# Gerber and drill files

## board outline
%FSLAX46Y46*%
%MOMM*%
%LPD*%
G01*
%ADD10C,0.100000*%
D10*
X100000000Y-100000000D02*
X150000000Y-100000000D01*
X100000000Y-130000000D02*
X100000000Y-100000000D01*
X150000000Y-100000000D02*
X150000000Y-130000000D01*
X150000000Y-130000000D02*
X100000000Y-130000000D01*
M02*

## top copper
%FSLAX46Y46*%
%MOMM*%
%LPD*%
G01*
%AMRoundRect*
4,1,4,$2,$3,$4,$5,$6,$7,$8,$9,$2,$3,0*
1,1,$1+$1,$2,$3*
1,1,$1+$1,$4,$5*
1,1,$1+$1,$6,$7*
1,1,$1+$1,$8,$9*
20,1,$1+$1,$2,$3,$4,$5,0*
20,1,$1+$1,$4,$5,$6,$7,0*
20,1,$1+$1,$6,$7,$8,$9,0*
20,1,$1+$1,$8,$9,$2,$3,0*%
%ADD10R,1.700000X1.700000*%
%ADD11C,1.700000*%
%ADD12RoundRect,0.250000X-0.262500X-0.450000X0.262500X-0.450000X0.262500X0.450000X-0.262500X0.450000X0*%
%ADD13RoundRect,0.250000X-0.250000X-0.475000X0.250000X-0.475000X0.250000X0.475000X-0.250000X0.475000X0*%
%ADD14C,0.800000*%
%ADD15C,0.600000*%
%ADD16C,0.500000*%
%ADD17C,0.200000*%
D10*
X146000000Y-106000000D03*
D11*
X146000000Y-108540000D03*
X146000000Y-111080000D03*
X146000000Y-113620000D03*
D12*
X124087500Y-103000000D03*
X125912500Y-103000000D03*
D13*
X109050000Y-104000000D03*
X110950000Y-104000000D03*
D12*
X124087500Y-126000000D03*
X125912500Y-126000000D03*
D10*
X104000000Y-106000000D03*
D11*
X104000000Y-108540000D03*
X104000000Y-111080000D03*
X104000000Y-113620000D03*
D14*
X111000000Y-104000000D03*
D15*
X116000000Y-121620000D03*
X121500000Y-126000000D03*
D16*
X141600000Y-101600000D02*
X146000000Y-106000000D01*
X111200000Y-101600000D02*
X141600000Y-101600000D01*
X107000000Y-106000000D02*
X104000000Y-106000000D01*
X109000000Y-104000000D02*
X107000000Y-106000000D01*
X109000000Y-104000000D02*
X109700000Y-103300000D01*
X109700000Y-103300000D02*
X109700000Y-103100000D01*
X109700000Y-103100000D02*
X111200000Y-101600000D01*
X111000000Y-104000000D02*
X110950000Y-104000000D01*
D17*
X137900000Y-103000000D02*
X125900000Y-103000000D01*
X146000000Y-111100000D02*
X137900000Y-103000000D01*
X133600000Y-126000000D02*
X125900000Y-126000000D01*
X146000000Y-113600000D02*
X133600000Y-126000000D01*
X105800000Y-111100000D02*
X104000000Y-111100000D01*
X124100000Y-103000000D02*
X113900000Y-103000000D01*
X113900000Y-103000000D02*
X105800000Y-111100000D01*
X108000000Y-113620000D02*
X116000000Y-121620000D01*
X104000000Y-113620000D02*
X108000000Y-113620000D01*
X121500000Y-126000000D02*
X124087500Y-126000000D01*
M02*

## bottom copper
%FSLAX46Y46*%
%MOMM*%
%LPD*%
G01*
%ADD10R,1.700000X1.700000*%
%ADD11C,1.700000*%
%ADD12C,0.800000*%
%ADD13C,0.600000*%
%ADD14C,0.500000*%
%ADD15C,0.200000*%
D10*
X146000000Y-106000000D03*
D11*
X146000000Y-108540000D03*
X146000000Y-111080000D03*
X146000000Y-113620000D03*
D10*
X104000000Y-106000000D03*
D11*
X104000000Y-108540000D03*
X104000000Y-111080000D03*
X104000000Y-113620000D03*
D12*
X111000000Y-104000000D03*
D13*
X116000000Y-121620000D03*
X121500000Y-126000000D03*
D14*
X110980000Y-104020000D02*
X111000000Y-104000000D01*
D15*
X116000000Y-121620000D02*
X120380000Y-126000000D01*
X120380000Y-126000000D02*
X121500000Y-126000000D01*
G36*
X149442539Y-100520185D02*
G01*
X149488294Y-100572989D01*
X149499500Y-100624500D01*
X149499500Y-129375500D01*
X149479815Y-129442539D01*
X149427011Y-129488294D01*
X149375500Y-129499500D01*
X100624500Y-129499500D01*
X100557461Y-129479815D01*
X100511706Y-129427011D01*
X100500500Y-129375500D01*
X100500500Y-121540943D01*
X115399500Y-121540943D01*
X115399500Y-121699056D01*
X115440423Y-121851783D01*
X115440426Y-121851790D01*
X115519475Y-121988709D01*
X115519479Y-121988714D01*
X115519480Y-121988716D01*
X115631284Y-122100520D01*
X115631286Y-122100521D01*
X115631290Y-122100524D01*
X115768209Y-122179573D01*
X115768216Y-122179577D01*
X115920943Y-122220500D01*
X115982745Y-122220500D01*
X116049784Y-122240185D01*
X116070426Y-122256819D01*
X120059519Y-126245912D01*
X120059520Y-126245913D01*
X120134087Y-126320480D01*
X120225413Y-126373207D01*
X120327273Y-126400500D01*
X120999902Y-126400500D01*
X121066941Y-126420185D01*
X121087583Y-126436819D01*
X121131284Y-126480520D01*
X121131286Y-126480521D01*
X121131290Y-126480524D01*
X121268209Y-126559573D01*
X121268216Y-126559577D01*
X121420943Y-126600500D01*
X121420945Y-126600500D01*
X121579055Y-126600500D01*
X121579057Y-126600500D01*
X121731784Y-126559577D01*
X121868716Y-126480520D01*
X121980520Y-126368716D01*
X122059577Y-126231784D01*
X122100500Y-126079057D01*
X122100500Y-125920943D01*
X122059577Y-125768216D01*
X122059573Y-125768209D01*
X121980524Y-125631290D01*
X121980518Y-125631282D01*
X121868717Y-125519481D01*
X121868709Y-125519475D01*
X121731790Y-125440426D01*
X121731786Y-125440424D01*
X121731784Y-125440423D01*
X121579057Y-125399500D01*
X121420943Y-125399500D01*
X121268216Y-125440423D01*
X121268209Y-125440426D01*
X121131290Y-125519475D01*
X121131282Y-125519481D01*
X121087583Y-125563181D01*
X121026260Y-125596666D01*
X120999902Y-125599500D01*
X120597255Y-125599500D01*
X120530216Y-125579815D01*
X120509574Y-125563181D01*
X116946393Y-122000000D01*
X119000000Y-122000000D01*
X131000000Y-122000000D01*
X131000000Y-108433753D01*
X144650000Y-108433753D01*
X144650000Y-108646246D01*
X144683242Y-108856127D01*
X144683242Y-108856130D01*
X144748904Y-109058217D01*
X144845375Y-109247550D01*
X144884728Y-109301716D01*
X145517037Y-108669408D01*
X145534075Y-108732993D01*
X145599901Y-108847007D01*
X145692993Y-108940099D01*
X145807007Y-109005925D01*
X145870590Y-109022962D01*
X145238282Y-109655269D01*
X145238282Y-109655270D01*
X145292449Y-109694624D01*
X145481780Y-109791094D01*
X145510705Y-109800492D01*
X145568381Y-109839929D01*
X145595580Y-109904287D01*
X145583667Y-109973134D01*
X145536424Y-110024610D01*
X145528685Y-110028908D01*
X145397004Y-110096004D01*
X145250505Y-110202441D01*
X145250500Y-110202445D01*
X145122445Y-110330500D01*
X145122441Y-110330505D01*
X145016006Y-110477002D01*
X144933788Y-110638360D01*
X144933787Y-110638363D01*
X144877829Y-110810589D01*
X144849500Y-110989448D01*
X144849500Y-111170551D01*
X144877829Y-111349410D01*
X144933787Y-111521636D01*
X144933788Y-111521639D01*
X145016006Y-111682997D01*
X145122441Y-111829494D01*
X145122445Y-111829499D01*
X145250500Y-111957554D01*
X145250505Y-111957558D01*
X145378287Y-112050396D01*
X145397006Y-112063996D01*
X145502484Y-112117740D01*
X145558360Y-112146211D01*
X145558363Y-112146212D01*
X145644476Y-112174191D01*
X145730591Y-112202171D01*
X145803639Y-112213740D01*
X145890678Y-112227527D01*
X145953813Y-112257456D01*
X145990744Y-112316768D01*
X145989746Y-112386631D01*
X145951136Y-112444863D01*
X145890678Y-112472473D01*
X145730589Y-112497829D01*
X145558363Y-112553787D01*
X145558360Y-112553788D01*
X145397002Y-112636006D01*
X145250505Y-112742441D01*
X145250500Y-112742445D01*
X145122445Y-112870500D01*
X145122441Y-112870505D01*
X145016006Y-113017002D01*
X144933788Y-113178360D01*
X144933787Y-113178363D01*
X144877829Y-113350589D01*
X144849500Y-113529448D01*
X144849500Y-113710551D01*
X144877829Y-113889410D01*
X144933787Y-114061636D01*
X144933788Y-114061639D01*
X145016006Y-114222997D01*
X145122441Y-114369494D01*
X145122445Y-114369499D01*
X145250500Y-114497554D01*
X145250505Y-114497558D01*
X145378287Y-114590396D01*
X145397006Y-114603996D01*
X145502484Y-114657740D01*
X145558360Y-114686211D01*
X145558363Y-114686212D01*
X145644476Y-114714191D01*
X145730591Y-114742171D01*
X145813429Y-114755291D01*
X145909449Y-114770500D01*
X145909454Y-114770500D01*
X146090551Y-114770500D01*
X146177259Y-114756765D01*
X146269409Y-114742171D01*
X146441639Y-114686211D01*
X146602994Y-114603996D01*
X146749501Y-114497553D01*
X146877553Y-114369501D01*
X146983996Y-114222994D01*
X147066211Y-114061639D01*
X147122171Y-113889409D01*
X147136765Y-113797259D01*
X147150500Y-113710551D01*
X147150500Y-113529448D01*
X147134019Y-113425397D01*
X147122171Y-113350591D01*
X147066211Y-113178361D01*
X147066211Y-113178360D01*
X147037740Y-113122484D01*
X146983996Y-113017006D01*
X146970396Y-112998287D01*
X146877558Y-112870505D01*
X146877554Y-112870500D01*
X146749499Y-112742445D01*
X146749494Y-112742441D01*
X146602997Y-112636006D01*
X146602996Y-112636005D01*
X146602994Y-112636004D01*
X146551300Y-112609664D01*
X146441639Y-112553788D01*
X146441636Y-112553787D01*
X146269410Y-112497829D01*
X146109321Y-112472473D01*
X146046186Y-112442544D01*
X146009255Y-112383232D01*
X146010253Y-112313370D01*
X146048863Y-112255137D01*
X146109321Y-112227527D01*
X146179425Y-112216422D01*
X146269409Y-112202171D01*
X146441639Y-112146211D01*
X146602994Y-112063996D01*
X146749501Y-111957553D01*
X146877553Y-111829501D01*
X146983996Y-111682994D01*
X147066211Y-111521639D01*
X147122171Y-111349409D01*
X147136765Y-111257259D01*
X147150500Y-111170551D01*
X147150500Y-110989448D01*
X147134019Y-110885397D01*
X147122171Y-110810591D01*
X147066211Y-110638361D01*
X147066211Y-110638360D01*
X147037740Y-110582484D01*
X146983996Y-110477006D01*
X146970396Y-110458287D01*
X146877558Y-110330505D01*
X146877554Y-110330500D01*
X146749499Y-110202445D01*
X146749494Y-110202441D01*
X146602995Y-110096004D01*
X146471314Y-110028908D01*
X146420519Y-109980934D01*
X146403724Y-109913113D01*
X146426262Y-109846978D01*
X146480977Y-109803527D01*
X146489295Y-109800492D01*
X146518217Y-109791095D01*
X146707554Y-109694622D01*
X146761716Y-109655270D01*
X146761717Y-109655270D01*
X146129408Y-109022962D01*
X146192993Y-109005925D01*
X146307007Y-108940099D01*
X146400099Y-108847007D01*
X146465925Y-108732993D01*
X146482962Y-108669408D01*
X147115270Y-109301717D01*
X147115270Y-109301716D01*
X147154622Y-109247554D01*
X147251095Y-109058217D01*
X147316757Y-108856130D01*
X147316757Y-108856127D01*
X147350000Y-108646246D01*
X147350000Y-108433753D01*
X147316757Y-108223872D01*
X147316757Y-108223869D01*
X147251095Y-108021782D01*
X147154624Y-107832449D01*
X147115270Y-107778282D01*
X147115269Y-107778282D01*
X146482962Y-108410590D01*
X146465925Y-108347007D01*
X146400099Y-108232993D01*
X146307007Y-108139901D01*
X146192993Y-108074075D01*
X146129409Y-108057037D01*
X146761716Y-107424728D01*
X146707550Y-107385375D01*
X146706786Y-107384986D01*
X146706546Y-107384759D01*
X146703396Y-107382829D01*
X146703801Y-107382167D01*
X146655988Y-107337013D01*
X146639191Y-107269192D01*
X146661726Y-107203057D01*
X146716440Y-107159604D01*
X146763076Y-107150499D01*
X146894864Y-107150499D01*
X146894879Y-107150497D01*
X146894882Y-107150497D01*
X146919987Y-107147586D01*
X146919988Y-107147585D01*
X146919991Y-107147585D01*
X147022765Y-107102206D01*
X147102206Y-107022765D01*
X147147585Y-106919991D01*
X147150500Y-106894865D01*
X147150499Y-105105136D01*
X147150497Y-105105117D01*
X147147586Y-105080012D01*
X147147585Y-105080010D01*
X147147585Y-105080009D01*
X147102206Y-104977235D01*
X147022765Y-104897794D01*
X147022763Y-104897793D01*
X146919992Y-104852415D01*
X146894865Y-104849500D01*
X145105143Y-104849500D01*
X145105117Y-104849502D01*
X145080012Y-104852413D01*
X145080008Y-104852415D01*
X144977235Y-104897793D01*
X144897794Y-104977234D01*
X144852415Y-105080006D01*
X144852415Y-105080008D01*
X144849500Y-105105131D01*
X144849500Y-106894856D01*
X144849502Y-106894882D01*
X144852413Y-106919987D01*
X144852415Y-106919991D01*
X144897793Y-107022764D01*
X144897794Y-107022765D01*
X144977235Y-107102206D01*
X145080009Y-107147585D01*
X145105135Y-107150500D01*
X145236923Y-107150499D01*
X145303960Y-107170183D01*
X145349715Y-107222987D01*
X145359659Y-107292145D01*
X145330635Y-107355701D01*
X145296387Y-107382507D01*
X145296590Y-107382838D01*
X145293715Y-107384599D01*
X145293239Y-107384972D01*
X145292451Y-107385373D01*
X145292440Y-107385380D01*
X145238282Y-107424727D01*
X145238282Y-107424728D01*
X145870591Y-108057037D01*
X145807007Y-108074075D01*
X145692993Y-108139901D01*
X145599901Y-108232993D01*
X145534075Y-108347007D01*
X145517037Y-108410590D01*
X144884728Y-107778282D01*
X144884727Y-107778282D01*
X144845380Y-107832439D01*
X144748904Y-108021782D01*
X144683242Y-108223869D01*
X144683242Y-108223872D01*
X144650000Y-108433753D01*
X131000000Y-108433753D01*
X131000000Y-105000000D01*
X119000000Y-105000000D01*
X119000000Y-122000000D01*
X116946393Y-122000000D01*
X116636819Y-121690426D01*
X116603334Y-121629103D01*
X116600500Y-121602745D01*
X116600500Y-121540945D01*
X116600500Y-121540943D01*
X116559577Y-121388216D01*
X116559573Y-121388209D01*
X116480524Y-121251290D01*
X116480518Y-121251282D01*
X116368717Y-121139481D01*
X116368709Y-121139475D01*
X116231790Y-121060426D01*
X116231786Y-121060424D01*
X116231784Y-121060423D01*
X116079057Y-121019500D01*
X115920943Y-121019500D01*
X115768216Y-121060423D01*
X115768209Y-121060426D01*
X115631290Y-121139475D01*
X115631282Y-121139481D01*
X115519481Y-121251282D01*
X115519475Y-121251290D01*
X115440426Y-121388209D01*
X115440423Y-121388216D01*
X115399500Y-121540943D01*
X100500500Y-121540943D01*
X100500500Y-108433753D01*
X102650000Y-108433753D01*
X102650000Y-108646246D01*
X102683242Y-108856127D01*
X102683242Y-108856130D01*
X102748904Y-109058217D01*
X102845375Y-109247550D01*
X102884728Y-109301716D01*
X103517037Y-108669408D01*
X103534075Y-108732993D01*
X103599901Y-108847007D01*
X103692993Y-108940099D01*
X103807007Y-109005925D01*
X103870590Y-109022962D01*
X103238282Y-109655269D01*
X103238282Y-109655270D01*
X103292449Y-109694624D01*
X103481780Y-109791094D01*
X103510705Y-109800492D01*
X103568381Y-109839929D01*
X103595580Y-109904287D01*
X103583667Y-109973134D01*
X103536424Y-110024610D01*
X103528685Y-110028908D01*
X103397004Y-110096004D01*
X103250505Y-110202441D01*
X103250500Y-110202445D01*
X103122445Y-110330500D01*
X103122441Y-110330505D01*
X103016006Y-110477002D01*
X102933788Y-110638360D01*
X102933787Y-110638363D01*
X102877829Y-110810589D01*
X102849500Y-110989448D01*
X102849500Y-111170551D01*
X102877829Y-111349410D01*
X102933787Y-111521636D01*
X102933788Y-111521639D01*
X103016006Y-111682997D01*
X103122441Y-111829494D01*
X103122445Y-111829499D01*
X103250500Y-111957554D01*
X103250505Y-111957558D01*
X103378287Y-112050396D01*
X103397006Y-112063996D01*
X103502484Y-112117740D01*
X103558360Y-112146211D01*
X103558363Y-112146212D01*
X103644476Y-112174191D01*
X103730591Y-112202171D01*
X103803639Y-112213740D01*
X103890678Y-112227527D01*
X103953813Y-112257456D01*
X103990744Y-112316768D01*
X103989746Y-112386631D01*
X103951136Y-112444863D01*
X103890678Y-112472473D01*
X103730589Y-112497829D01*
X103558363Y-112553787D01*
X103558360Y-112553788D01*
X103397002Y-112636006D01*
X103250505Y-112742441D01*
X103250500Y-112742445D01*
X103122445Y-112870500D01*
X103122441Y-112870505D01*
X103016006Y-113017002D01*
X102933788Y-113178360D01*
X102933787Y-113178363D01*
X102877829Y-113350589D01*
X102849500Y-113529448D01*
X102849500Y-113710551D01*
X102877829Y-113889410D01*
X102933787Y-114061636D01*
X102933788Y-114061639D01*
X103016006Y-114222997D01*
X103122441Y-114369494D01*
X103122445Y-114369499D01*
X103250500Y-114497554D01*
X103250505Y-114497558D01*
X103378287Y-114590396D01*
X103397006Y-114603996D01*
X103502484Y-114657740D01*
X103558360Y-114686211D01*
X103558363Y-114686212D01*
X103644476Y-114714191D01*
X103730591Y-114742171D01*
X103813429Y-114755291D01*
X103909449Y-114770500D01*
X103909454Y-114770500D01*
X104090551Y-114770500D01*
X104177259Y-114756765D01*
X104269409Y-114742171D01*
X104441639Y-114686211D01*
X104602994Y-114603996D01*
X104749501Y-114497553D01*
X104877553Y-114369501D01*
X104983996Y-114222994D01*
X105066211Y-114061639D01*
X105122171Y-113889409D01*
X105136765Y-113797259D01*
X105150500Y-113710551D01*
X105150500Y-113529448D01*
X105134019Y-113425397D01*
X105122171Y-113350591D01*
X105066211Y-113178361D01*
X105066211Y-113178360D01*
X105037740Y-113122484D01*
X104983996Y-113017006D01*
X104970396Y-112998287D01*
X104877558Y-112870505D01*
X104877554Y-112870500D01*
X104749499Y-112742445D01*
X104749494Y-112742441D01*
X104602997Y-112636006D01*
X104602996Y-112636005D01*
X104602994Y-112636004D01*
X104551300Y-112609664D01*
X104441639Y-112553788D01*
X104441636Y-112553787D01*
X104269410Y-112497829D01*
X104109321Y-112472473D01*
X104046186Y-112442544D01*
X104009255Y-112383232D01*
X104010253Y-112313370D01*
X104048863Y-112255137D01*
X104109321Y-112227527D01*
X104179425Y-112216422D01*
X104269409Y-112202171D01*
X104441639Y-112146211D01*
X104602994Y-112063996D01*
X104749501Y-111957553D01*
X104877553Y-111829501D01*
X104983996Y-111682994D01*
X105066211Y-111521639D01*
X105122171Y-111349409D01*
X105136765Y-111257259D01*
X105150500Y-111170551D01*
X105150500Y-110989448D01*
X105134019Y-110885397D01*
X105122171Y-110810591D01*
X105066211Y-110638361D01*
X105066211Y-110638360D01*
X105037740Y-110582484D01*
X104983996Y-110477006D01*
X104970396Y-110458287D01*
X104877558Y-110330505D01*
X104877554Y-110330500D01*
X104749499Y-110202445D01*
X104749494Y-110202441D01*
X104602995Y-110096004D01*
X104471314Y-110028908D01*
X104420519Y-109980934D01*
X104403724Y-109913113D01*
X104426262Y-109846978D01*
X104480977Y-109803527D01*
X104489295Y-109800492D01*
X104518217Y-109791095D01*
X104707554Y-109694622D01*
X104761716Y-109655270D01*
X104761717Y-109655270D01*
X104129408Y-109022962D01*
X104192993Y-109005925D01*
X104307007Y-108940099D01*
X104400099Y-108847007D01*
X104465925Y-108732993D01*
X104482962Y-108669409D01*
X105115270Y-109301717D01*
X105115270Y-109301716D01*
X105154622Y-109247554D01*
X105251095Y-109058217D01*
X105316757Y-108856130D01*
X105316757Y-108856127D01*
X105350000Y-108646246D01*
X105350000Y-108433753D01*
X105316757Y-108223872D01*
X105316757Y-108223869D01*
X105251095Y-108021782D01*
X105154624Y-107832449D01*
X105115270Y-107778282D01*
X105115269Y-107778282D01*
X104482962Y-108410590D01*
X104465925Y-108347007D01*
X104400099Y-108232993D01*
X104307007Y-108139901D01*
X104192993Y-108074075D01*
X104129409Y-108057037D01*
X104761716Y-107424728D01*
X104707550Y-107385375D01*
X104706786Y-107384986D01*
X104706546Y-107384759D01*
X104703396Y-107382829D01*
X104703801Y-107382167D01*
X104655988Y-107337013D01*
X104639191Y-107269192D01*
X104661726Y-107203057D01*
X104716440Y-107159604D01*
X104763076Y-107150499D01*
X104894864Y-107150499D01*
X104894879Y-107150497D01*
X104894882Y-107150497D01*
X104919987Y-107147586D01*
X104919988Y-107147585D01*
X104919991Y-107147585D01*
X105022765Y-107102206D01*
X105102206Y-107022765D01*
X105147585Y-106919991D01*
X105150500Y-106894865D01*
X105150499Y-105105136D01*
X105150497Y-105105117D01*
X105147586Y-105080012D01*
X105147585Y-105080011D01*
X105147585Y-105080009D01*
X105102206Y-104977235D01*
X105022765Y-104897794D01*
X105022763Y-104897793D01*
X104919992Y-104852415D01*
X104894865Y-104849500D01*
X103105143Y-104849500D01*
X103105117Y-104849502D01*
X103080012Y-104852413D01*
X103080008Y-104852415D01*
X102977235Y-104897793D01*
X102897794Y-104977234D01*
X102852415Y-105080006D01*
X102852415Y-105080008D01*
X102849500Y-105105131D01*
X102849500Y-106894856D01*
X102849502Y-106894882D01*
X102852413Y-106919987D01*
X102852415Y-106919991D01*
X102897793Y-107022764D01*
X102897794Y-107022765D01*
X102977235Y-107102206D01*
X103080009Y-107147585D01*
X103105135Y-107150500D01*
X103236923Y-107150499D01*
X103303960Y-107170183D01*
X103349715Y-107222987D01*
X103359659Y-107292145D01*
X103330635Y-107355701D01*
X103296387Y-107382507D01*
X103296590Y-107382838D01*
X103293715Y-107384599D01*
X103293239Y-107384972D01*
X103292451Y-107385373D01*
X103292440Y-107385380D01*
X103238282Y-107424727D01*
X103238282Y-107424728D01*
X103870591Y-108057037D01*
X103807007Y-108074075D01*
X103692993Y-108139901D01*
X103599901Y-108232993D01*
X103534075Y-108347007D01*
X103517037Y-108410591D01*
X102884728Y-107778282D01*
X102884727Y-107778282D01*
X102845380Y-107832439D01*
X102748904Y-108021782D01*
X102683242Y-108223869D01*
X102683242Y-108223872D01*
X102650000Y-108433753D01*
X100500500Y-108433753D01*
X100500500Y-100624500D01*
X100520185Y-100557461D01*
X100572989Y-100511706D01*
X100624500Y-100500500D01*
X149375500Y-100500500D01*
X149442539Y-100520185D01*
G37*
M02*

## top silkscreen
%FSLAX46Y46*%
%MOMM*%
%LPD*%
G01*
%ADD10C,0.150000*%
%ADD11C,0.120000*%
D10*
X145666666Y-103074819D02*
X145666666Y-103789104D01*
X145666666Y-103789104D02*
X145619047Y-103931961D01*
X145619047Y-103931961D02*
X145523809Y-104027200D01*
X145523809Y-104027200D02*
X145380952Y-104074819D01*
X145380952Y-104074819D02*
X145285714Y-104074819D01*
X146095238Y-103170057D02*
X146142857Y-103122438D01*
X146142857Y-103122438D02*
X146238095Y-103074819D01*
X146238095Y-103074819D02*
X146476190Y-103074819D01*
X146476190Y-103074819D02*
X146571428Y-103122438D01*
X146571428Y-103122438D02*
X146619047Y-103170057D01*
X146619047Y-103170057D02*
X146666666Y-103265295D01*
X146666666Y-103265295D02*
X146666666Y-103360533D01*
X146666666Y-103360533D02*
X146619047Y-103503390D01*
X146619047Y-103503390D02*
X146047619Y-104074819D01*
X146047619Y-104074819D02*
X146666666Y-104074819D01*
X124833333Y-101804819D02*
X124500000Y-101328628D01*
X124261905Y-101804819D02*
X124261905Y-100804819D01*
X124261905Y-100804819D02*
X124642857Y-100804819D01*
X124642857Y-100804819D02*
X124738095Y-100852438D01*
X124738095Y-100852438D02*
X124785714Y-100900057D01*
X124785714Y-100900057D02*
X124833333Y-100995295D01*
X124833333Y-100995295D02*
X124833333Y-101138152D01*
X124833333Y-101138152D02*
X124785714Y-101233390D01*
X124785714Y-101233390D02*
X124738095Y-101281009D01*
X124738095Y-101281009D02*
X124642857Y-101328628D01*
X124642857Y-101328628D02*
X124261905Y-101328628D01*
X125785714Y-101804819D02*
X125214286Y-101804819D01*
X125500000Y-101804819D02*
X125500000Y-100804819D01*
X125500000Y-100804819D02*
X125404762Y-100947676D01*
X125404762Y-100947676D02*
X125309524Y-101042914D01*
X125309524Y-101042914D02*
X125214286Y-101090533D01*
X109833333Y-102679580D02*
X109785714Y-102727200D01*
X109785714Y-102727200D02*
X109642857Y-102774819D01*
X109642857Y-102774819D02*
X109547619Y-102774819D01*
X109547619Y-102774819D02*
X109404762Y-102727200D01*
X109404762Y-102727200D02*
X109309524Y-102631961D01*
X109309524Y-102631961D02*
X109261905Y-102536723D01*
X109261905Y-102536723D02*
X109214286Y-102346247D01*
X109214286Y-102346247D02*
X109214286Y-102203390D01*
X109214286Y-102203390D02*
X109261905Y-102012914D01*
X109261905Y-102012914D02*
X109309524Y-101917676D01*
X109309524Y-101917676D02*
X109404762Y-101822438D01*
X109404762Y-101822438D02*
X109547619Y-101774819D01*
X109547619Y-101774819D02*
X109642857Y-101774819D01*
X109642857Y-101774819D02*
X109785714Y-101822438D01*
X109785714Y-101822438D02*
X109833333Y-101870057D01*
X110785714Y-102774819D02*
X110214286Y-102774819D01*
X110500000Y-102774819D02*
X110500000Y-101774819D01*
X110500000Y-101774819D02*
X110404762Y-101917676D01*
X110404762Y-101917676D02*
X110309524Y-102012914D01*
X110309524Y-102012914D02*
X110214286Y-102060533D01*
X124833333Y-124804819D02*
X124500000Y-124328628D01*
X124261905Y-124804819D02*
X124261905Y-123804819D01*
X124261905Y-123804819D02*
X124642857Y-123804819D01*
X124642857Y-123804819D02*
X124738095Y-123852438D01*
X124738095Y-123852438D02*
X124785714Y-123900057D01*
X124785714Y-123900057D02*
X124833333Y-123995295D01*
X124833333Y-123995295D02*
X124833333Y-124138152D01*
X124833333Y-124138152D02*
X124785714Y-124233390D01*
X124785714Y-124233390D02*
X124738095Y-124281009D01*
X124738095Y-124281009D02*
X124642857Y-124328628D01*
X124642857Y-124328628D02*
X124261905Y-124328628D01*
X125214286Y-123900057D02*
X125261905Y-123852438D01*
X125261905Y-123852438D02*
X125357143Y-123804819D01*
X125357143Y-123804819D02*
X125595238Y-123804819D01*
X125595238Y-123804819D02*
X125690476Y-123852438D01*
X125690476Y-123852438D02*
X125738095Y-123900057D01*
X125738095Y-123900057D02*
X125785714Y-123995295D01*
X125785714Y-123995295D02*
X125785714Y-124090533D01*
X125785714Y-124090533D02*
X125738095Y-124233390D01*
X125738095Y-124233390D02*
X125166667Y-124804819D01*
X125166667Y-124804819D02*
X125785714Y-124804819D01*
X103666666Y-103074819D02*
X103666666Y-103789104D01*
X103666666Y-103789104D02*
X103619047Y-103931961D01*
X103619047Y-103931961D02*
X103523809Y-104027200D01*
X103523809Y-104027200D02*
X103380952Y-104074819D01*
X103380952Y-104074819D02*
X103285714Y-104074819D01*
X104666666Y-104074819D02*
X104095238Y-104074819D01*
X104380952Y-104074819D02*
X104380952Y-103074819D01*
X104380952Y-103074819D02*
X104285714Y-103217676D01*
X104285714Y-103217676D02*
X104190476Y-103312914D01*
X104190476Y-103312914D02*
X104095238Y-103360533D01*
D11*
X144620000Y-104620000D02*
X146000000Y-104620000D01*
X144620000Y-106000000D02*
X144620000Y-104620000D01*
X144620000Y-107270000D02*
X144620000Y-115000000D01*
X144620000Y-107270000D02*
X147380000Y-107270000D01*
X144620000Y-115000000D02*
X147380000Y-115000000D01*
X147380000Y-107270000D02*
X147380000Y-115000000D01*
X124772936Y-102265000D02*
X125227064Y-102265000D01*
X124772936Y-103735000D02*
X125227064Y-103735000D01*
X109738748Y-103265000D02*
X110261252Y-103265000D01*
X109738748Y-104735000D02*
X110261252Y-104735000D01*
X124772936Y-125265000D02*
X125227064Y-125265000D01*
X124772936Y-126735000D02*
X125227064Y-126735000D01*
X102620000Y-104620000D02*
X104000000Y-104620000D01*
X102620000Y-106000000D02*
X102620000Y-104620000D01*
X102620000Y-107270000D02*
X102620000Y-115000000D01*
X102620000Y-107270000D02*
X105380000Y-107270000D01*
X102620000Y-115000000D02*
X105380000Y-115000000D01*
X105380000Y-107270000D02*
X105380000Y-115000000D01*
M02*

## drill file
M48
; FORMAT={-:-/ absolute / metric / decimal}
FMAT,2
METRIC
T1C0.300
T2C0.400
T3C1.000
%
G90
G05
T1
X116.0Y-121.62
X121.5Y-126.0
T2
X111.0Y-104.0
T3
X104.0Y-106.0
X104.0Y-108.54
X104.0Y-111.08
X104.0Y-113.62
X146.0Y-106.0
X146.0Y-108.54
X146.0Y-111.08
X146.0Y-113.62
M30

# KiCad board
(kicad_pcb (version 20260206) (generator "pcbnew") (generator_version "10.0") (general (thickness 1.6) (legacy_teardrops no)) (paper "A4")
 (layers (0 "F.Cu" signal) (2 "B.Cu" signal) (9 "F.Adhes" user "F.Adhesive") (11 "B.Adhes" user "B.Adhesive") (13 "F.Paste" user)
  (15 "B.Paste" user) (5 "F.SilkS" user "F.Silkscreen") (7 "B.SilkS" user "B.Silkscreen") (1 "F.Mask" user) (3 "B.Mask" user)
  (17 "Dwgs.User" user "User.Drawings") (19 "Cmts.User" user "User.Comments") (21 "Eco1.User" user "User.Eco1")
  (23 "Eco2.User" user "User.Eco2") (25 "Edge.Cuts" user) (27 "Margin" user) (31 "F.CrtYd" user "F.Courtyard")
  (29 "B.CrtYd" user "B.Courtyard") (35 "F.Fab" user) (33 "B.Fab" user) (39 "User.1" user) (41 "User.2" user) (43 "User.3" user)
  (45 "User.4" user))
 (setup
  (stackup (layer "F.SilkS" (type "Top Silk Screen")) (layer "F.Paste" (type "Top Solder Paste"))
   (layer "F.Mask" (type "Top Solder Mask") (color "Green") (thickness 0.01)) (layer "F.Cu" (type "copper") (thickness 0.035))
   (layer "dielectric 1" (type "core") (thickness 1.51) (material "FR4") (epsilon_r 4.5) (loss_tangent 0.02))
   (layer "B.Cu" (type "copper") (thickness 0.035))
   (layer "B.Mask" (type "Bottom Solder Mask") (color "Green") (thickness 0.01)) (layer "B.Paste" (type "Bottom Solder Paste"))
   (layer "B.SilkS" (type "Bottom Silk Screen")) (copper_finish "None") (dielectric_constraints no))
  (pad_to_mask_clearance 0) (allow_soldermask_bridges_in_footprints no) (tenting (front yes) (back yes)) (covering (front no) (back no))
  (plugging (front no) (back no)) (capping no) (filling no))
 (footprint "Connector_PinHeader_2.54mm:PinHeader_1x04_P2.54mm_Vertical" (layer "F.Cu") (at 146 106)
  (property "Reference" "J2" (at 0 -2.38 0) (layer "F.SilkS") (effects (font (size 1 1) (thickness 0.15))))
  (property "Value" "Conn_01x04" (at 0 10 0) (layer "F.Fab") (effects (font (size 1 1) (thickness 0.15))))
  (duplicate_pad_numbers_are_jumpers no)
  (fp_line (start -1.38 -1.38) (end 0 -1.38) (stroke (width 0.12) (type solid)) (layer "F.SilkS"))
  (fp_line (start -1.38 0) (end -1.38 -1.38) (stroke (width 0.12) (type solid)) (layer "F.SilkS"))
  (fp_line (start -1.38 1.27) (end -1.38 9) (stroke (width 0.12) (type solid)) (layer "F.SilkS"))
  (fp_line (start -1.38 1.27) (end 1.38 1.27) (stroke (width 0.12) (type solid)) (layer "F.SilkS"))
  (fp_line (start -1.38 9) (end 1.38 9) (stroke (width 0.12) (type solid)) (layer "F.SilkS"))
  (fp_line (start 1.38 1.27) (end 1.38 9) (stroke (width 0.12) (type solid)) (layer "F.SilkS"))
  (pad "1" thru_hole rect (at 0 0) (size 1.7 1.7) (drill 1) (layers "*.Cu" "*.Mask") (remove_unused_layers no) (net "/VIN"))
  (pad "2" thru_hole circle (at 0 2.54) (size 1.7 1.7) (drill 1) (layers "*.Cu" "*.Mask") (remove_unused_layers no) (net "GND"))
  (pad "3" thru_hole circle (at 0 5.08) (size 1.7 1.7) (drill 1) (layers "*.Cu" "*.Mask") (remove_unused_layers no) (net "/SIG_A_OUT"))
  (pad "4" thru_hole circle (at 0 7.62) (size 1.7 1.7) (drill 1) (layers "*.Cu" "*.Mask") (remove_unused_layers no) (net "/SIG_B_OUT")))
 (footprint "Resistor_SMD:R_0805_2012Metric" (layer "F.Cu") (at 125 103)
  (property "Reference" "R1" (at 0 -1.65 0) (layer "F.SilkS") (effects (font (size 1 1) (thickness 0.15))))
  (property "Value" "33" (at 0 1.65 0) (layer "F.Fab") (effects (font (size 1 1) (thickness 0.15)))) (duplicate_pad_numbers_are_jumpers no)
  (fp_line (start -0.227064 -0.735) (end 0.227064 -0.735) (stroke (width 0.12) (type solid)) (layer "F.SilkS"))
  (fp_line (start -0.227064 0.735) (end 0.227064 0.735) (stroke (width 0.12) (type solid)) (layer "F.SilkS"))
  (pad "1" smd roundrect (at -0.9125 0) (size 1.025 1.4) (layers "F.Cu" "F.Mask" "F.Paste") (roundrect_rratio 0.243902) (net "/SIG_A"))
  (pad "2" smd roundrect (at 0.9125 0) (size 1.025 1.4) (layers "F.Cu" "F.Mask" "F.Paste") (roundrect_rratio 0.243902) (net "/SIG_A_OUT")))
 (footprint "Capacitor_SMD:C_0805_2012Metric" (layer "F.Cu") (at 110 104)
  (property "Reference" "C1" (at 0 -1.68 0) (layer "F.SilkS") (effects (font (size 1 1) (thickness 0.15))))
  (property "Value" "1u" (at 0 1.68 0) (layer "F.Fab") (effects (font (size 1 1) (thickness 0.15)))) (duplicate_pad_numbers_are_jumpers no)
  (fp_line (start -0.261252 -0.735) (end 0.261252 -0.735) (stroke (width 0.12) (type solid)) (layer "F.SilkS"))
  (fp_line (start -0.261252 0.735) (end 0.261252 0.735) (stroke (width 0.12) (type solid)) (layer "F.SilkS"))
  (pad "1" smd roundrect (at -0.95 0) (size 1 1.45) (layers "F.Cu" "F.Mask" "F.Paste") (roundrect_rratio 0.25) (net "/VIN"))
  (pad "2" smd roundrect (at 0.95 0) (size 1 1.45) (layers "F.Cu" "F.Mask" "F.Paste") (roundrect_rratio 0.25) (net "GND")))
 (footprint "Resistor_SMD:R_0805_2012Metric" (layer "F.Cu") (at 125 126)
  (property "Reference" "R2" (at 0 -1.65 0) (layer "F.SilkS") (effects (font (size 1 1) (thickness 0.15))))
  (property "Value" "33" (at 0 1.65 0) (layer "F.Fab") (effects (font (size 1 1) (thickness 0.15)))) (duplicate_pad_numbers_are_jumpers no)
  (fp_line (start -0.227064 -0.735) (end 0.227064 -0.735) (stroke (width 0.12) (type solid)) (layer "F.SilkS"))
  (fp_line (start -0.227064 0.735) (end 0.227064 0.735) (stroke (width 0.12) (type solid)) (layer "F.SilkS"))
  (pad "1" smd roundrect (at -0.9125 0) (size 1.025 1.4) (layers "F.Cu" "F.Mask" "F.Paste") (roundrect_rratio 0.243902) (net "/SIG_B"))
  (pad "2" smd roundrect (at 0.9125 0) (size 1.025 1.4) (layers "F.Cu" "F.Mask" "F.Paste") (roundrect_rratio 0.243902) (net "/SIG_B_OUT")))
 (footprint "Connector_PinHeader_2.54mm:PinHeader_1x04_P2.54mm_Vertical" (layer "F.Cu") (at 104 106)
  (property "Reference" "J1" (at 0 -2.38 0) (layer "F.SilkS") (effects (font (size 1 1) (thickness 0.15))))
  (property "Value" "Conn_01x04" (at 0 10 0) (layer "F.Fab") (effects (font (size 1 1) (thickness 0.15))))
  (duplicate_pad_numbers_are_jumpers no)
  (fp_line (start -1.38 -1.38) (end 0 -1.38) (stroke (width 0.12) (type solid)) (layer "F.SilkS"))
  (fp_line (start -1.38 0) (end -1.38 -1.38) (stroke (width 0.12) (type solid)) (layer "F.SilkS"))
  (fp_line (start -1.38 1.27) (end -1.38 9) (stroke (width 0.12) (type solid)) (layer "F.SilkS"))
  (fp_line (start -1.38 1.27) (end 1.38 1.27) (stroke (width 0.12) (type solid)) (layer "F.SilkS"))
  (fp_line (start -1.38 9) (end 1.38 9) (stroke (width 0.12) (type solid)) (layer "F.SilkS"))
  (fp_line (start 1.38 1.27) (end 1.38 9) (stroke (width 0.12) (type solid)) (layer "F.SilkS"))
  (pad "1" thru_hole rect (at 0 0) (size 1.7 1.7) (drill 1) (layers "*.Cu" "*.Mask") (remove_unused_layers no) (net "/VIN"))
  (pad "2" thru_hole circle (at 0 2.54) (size 1.7 1.7) (drill 1) (layers "*.Cu" "*.Mask") (remove_unused_layers no) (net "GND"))
  (pad "3" thru_hole circle (at 0 5.08) (size 1.7 1.7) (drill 1) (layers "*.Cu" "*.Mask") (remove_unused_layers no) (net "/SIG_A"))
  (pad "4" thru_hole circle (at 0 7.62) (size 1.7 1.7) (drill 1) (layers "*.Cu" "*.Mask") (remove_unused_layers no) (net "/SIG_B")))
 (gr_line (start 100 100) (end 150 100) (stroke (width 0.1) (type default)) (layer "Edge.Cuts"))
 (gr_line (start 100 130) (end 100 100) (stroke (width 0.1) (type default)) (layer "Edge.Cuts"))
 (gr_line (start 150 100) (end 150 130) (stroke (width 0.1) (type default)) (layer "Edge.Cuts"))
 (gr_line (start 150 130) (end 100 130) (stroke (width 0.1) (type default)) (layer "Edge.Cuts"))
 (segment (start 141.6 101.6) (end 146 106) (width 0.5) (layer "F.Cu") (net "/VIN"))
 (segment (start 111.2 101.6) (end 141.6 101.6) (width 0.5) (layer "F.Cu") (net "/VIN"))
 (segment (start 107 106) (end 104 106) (width 0.5) (layer "F.Cu") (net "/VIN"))
 (segment (start 109 104) (end 107 106) (width 0.5) (layer "F.Cu") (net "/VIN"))
 (segment (start 109 104) (end 109.7 103.3) (width 0.5) (layer "F.Cu") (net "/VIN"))
 (segment (start 109.7 103.3) (end 109.7 103.1) (width 0.5) (layer "F.Cu") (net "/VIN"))
 (segment (start 109.7 103.1) (end 111.2 101.6) (width 0.5) (layer "F.Cu") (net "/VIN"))
 (segment (start 111 104) (end 110.95 104) (width 0.5) (layer "F.Cu") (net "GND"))
 (via (at 111 104) (size 0.8) (drill 0.4) (layers "F.Cu" "B.Cu") (capping yes) (filling yes) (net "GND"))
 (segment (start 110.98 104.02) (end 111 104) (width 0.5) (layer "B.Cu") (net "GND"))
 (segment (start 137.9 103) (end 125.9 103) (width 0.2) (layer "F.Cu") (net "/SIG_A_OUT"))
 (segment (start 146 111.1) (end 137.9 103) (width 0.2) (layer "F.Cu") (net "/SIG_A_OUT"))
 (segment (start 133.6 126) (end 125.9 126) (width 0.2) (layer "F.Cu") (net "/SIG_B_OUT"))
 (segment (start 146 113.6) (end 133.6 126) (width 0.2) (layer "F.Cu") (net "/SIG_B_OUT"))
 (segment (start 105.8 111.1) (end 104 111.1) (width 0.2) (layer "F.Cu") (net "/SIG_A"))
 (segment (start 124.1 103) (end 113.9 103) (width 0.2) (layer "F.Cu") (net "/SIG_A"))
 (segment (start 113.9 103) (end 105.8 111.1) (width 0.2) (layer "F.Cu") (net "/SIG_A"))
 (segment (start 108 113.62) (end 116 121.62) (width 0.2) (locked yes) (layer "F.Cu") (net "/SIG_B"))
 (segment (start 104 113.62) (end 108 113.62) (width 0.2) (locked yes) (layer "F.Cu") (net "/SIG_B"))
 (segment (start 121.5 126) (end 124.0875 126) (width 0.2) (locked yes) (layer "F.Cu") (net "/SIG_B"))
 (via (at 116 121.62) (size 0.6) (drill 0.3) (layers "F.Cu" "B.Cu") (locked yes) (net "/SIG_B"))
 (via (at 121.5 126) (size 0.6) (drill 0.3) (layers "F.Cu" "B.Cu") (locked yes) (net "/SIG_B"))
 (segment (start 116 121.62) (end 120.38 126) (width 0.2) (locked yes) (layer "B.Cu") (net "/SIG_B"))
 (segment (start 120.38 126) (end 121.5 126) (width 0.2) (locked yes) (layer "B.Cu") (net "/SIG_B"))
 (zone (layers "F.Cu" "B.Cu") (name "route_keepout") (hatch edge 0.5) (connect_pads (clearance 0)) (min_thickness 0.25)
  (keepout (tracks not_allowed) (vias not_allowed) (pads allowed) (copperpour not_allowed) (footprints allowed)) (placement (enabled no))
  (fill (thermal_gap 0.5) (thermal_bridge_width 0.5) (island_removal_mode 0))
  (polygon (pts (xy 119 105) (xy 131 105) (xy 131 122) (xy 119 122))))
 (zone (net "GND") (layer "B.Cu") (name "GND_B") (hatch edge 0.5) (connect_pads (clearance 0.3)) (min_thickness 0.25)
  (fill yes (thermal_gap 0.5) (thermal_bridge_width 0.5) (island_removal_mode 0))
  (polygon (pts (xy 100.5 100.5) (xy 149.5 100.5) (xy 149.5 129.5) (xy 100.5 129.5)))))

